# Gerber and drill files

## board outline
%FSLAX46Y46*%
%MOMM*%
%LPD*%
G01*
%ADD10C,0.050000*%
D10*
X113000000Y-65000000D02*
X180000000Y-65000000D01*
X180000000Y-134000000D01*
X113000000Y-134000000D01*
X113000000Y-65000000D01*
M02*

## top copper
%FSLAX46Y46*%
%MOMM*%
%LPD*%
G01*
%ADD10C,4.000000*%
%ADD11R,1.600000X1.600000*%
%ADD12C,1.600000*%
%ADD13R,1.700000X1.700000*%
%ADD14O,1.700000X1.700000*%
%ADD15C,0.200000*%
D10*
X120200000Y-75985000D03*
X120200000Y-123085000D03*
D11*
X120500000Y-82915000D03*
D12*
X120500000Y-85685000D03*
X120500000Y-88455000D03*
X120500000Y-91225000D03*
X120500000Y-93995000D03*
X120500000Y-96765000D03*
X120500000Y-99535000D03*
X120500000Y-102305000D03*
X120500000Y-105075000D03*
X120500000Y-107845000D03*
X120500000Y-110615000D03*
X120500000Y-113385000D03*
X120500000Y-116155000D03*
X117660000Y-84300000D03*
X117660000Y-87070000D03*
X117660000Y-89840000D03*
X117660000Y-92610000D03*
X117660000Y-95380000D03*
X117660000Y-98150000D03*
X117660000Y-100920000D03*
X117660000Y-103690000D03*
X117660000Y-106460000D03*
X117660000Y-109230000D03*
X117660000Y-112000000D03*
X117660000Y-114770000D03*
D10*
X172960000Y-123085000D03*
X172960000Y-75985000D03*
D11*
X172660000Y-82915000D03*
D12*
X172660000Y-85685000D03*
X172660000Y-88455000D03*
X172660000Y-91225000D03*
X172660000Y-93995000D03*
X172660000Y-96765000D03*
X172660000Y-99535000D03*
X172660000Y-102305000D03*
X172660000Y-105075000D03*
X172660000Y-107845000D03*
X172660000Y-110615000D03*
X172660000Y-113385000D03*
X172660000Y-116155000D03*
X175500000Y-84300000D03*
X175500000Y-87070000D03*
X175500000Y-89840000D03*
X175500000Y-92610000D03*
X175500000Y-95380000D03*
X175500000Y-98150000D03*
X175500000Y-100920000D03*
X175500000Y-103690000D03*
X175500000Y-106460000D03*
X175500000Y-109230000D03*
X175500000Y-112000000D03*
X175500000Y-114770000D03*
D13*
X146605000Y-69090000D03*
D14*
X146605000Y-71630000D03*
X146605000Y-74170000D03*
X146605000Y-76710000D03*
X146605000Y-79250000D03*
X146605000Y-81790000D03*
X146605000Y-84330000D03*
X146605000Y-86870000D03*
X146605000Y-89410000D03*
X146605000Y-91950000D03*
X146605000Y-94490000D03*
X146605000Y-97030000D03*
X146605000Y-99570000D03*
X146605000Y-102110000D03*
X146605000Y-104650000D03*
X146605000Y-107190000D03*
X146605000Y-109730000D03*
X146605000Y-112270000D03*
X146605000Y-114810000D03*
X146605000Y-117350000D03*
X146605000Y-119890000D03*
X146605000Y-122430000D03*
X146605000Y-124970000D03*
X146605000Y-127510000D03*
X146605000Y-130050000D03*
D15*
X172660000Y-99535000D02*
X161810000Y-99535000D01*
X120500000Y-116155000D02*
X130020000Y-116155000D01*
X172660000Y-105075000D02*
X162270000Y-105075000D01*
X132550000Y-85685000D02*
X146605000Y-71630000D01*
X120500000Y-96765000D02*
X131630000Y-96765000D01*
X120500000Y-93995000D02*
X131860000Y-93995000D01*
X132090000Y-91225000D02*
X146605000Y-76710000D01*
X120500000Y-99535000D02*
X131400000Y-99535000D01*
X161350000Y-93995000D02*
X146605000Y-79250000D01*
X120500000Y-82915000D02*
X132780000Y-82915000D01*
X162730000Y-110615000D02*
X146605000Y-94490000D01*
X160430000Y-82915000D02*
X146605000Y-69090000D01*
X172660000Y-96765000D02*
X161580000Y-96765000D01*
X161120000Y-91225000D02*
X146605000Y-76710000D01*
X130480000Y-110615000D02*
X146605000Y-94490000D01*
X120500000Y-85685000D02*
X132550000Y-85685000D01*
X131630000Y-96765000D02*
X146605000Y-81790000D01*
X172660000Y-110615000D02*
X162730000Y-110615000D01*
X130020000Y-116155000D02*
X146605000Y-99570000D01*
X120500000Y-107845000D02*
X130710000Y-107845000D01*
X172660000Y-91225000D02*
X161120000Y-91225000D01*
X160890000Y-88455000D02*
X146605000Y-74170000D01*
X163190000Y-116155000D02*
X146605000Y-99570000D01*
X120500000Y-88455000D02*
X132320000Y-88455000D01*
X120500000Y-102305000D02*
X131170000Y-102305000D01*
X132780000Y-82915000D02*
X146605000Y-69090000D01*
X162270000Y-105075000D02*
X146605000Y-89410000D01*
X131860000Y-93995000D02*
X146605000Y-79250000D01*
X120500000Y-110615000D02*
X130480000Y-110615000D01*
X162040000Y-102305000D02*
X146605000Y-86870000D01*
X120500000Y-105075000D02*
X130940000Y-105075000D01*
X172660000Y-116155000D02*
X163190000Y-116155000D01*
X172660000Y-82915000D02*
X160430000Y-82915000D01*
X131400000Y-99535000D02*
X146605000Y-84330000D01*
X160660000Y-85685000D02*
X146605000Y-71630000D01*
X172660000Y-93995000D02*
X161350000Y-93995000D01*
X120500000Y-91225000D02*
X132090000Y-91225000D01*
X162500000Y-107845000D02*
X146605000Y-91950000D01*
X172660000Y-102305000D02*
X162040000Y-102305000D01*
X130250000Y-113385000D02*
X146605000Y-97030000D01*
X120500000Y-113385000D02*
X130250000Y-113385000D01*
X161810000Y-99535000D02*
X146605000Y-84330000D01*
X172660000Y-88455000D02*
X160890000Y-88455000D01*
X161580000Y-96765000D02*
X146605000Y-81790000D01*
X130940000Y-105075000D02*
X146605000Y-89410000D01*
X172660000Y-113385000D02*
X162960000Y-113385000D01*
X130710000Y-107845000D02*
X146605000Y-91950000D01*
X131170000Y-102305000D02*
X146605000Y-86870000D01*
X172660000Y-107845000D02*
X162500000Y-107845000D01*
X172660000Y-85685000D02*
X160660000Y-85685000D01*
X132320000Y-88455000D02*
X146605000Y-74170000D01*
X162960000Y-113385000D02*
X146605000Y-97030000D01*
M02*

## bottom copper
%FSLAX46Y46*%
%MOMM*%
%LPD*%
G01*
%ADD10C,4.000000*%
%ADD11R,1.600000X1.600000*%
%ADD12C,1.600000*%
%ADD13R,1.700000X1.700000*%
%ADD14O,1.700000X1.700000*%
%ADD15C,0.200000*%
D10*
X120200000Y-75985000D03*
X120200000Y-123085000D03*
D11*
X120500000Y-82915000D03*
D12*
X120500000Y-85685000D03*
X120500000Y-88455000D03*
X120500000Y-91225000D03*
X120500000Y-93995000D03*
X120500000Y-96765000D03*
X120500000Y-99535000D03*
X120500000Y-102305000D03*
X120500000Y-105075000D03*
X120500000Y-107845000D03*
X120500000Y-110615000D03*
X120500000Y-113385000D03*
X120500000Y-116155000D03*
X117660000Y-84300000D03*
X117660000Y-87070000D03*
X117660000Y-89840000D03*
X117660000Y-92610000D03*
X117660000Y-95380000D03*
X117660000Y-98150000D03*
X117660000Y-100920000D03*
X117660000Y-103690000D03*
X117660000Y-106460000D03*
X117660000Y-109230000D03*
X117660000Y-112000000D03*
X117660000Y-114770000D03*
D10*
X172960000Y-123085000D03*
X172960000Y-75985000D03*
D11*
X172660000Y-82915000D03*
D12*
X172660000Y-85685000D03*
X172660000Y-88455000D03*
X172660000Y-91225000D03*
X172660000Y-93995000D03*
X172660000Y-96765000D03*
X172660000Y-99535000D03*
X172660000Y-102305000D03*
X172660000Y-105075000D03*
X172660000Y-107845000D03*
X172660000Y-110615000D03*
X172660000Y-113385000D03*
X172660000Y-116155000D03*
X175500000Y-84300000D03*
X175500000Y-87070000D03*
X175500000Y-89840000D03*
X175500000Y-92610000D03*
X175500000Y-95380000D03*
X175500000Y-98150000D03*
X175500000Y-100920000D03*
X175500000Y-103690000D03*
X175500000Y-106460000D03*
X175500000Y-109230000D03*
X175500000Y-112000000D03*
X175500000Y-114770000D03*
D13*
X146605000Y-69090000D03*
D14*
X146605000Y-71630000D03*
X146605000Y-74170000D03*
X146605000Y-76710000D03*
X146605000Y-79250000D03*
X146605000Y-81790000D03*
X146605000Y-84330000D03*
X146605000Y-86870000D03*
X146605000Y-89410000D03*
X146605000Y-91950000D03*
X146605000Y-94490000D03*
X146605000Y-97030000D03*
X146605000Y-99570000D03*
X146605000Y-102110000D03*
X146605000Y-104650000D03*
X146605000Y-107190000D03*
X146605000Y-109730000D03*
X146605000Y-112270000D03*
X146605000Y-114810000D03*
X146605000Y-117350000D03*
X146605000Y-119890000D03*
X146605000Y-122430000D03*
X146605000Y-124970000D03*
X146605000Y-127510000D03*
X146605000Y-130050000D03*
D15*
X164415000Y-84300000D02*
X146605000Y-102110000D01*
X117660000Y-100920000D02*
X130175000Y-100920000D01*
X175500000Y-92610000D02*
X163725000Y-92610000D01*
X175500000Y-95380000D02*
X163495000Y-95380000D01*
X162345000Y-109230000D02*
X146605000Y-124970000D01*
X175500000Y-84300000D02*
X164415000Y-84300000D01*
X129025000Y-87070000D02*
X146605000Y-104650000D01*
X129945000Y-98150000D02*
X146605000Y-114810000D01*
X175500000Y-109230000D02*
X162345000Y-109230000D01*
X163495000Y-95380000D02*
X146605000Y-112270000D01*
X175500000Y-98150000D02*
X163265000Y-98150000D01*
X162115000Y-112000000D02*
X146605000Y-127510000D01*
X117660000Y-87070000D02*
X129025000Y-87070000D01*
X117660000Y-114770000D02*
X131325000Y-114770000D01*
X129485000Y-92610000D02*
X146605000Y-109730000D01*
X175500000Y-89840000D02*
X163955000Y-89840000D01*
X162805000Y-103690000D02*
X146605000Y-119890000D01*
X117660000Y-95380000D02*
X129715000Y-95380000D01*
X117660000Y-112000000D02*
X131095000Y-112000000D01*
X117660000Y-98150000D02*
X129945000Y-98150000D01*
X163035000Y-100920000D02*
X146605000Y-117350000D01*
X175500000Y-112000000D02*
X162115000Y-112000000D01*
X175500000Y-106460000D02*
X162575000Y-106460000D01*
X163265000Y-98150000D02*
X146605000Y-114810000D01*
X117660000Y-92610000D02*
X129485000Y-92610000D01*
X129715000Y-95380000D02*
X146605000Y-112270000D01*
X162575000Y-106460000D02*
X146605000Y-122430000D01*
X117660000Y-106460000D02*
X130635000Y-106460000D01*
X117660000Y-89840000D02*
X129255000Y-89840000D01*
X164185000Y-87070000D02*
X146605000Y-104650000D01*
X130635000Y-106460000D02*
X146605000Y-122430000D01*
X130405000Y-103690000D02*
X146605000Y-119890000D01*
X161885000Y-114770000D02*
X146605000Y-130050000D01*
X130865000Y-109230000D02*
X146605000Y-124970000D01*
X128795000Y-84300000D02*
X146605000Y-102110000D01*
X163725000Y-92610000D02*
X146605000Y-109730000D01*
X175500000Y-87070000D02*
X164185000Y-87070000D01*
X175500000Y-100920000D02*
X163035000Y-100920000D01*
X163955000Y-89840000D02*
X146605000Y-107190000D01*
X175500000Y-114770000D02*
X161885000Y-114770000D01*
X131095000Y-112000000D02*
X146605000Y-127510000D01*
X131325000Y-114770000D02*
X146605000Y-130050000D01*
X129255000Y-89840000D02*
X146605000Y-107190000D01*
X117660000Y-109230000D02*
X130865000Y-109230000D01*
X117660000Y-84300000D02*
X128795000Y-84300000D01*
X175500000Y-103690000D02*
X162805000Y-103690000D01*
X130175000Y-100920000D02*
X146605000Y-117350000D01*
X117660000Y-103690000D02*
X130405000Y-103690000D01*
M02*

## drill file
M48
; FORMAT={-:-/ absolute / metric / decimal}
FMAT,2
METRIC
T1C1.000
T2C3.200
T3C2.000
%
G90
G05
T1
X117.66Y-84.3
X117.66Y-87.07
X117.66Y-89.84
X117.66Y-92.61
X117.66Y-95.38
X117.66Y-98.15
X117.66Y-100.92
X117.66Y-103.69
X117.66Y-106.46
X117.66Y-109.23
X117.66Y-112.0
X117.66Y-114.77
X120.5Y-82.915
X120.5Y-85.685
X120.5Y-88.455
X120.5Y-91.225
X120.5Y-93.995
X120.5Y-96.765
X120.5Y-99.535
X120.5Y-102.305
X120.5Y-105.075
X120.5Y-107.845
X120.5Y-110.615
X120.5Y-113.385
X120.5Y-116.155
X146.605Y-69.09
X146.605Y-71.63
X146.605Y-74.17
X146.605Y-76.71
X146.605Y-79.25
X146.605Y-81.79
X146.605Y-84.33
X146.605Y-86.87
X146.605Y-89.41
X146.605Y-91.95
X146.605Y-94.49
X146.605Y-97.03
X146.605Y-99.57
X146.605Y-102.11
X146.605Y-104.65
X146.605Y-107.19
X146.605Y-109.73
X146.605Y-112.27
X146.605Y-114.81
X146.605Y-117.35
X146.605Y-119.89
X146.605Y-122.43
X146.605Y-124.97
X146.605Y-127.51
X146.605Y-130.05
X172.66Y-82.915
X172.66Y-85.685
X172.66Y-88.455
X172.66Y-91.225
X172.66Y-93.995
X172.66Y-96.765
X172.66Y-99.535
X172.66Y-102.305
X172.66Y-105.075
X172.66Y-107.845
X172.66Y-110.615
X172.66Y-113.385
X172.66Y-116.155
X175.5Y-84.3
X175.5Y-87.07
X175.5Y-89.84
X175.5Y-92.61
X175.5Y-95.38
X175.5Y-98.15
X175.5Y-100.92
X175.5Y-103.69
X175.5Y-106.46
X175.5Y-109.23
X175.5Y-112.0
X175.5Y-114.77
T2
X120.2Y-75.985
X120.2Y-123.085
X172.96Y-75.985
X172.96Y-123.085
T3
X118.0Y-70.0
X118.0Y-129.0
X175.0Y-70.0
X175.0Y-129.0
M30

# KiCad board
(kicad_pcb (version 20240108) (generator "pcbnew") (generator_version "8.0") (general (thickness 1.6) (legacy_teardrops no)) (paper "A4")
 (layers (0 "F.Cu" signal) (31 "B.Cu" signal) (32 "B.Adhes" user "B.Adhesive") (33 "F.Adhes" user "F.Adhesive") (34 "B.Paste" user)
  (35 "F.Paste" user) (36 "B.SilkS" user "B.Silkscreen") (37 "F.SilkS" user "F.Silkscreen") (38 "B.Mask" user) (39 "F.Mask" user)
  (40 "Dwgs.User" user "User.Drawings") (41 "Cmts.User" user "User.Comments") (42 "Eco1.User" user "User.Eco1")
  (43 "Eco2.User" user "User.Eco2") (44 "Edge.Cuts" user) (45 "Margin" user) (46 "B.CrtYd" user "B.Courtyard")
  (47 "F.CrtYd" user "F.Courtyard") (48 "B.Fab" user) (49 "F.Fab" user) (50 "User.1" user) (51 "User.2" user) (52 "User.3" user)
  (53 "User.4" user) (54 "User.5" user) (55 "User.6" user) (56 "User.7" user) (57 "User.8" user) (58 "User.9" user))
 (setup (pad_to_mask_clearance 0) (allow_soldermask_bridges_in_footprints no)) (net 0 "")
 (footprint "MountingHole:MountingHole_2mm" (layer "F.Cu") (at 175 70)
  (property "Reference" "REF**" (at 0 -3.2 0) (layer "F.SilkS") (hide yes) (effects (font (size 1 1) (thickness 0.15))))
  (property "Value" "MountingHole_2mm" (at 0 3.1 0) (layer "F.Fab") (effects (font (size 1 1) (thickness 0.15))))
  (pad "" np_thru_hole circle (at 0 0) (size 2 2) (drill 2) (layers "*.Cu" "*.Mask")))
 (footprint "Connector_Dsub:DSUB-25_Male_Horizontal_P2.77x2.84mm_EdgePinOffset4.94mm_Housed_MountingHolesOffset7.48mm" (layer "F.Cu")
  (at 120.5 82.915 -90)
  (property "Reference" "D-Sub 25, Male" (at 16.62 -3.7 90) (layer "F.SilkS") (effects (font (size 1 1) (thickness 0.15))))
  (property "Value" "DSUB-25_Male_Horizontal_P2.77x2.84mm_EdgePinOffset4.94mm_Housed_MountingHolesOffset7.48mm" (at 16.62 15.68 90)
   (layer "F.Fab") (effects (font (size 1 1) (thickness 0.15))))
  (pad "0" thru_hole circle (at -6.93 0.3 270) (size 4 4) (drill 3.2) (layers "*.Cu" "*.Mask") (remove_unused_layers no))
  (pad "0" thru_hole circle (at 40.17 0.3 270) (size 4 4) (drill 3.2) (layers "*.Cu" "*.Mask") (remove_unused_layers no))
  (pad "1" thru_hole rect (at 0 0 270) (size 1.6 1.6) (drill 1) (layers "*.Cu" "*.Mask") (remove_unused_layers no))
  (pad "2" thru_hole circle (at 2.77 0 270) (size 1.6 1.6) (drill 1) (layers "*.Cu" "*.Mask") (remove_unused_layers no))
  (pad "3" thru_hole circle (at 5.54 0 270) (size 1.6 1.6) (drill 1) (layers "*.Cu" "*.Mask") (remove_unused_layers no))
  (pad "4" thru_hole circle (at 8.31 0 270) (size 1.6 1.6) (drill 1) (layers "*.Cu" "*.Mask") (remove_unused_layers no))
  (pad "5" thru_hole circle (at 11.08 0 270) (size 1.6 1.6) (drill 1) (layers "*.Cu" "*.Mask") (remove_unused_layers no))
  (pad "6" thru_hole circle (at 13.85 0 270) (size 1.6 1.6) (drill 1) (layers "*.Cu" "*.Mask") (remove_unused_layers no))
  (pad "7" thru_hole circle (at 16.62 0 270) (size 1.6 1.6) (drill 1) (layers "*.Cu" "*.Mask") (remove_unused_layers no))
  (pad "8" thru_hole circle (at 19.39 0 270) (size 1.6 1.6) (drill 1) (layers "*.Cu" "*.Mask") (remove_unused_layers no))
  (pad "9" thru_hole circle (at 22.16 0 270) (size 1.6 1.6) (drill 1) (layers "*.Cu" "*.Mask") (remove_unused_layers no))
  (pad "10" thru_hole circle (at 24.93 0 270) (size 1.6 1.6) (drill 1) (layers "*.Cu" "*.Mask") (remove_unused_layers no))
  (pad "11" thru_hole circle (at 27.7 0 270) (size 1.6 1.6) (drill 1) (layers "*.Cu" "*.Mask") (remove_unused_layers no))
  (pad "12" thru_hole circle (at 30.47 0 270) (size 1.6 1.6) (drill 1) (layers "*.Cu" "*.Mask") (remove_unused_layers no))
  (pad "13" thru_hole circle (at 33.24 0 270) (size 1.6 1.6) (drill 1) (layers "*.Cu" "*.Mask") (remove_unused_layers no))
  (pad "14" thru_hole circle (at 1.385 2.84 270) (size 1.6 1.6) (drill 1) (layers "*.Cu" "*.Mask") (remove_unused_layers no))
  (pad "15" thru_hole circle (at 4.155 2.84 270) (size 1.6 1.6) (drill 1) (layers "*.Cu" "*.Mask") (remove_unused_layers no))
  (pad "16" thru_hole circle (at 6.925 2.84 270) (size 1.6 1.6) (drill 1) (layers "*.Cu" "*.Mask") (remove_unused_layers no))
  (pad "17" thru_hole circle (at 9.695 2.84 270) (size 1.6 1.6) (drill 1) (layers "*.Cu" "*.Mask") (remove_unused_layers no))
  (pad "18" thru_hole circle (at 12.465 2.84 270) (size 1.6 1.6) (drill 1) (layers "*.Cu" "*.Mask") (remove_unused_layers no))
  (pad "19" thru_hole circle (at 15.235 2.84 270) (size 1.6 1.6) (drill 1) (layers "*.Cu" "*.Mask") (remove_unused_layers no))
  (pad "20" thru_hole circle (at 18.005 2.84 270) (size 1.6 1.6) (drill 1) (layers "*.Cu" "*.Mask") (remove_unused_layers no))
  (pad "21" thru_hole circle (at 20.775 2.84 270) (size 1.6 1.6) (drill 1) (layers "*.Cu" "*.Mask") (remove_unused_layers no))
  (pad "22" thru_hole circle (at 23.545 2.84 270) (size 1.6 1.6) (drill 1) (layers "*.Cu" "*.Mask") (remove_unused_layers no))
  (pad "23" thru_hole circle (at 26.315 2.84 270) (size 1.6 1.6) (drill 1) (layers "*.Cu" "*.Mask") (remove_unused_layers no))
  (pad "24" thru_hole circle (at 29.085 2.84 270) (size 1.6 1.6) (drill 1) (layers "*.Cu" "*.Mask") (remove_unused_layers no))
  (pad "25" thru_hole circle (at 31.855 2.84 270) (size 1.6 1.6) (drill 1) (layers "*.Cu" "*.Mask") (remove_unused_layers no)))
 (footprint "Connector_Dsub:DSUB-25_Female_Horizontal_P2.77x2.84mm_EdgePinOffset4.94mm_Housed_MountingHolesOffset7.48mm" (layer "F.Cu")
  (at 172.66 82.915 90)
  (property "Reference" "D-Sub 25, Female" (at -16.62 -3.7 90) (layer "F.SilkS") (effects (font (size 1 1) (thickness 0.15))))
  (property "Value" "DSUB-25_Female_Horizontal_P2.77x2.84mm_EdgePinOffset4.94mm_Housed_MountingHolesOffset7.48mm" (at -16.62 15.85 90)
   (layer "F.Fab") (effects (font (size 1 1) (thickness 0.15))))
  (pad "0" thru_hole circle (at -40.17 0.3 90) (size 4 4) (drill 3.2) (layers "*.Cu" "*.Mask") (remove_unused_layers no))
  (pad "0" thru_hole circle (at 6.93 0.3 90) (size 4 4) (drill 3.2) (layers "*.Cu" "*.Mask") (remove_unused_layers no))
  (pad "1" thru_hole rect (at 0 0 90) (size 1.6 1.6) (drill 1) (layers "*.Cu" "*.Mask") (remove_unused_layers no))
  (pad "2" thru_hole circle (at -2.77 0 90) (size 1.6 1.6) (drill 1) (layers "*.Cu" "*.Mask") (remove_unused_layers no))
  (pad "3" thru_hole circle (at -5.54 0 90) (size 1.6 1.6) (drill 1) (layers "*.Cu" "*.Mask") (remove_unused_layers no))
  (pad "4" thru_hole circle (at -8.31 0 90) (size 1.6 1.6) (drill 1) (layers "*.Cu" "*.Mask") (remove_unused_layers no))
  (pad "5" thru_hole circle (at -11.08 0 90) (size 1.6 1.6) (drill 1) (layers "*.Cu" "*.Mask") (remove_unused_layers no))
  (pad "6" thru_hole circle (at -13.85 0 90) (size 1.6 1.6) (drill 1) (layers "*.Cu" "*.Mask") (remove_unused_layers no))
  (pad "7" thru_hole circle (at -16.62 0 90) (size 1.6 1.6) (drill 1) (layers "*.Cu" "*.Mask") (remove_unused_layers no))
  (pad "8" thru_hole circle (at -19.39 0 90) (size 1.6 1.6) (drill 1) (layers "*.Cu" "*.Mask") (remove_unused_layers no))
  (pad "9" thru_hole circle (at -22.16 0 90) (size 1.6 1.6) (drill 1) (layers "*.Cu" "*.Mask") (remove_unused_layers no))
  (pad "10" thru_hole circle (at -24.93 0 90) (size 1.6 1.6) (drill 1) (layers "*.Cu" "*.Mask") (remove_unused_layers no))
  (pad "11" thru_hole circle (at -27.7 0 90) (size 1.6 1.6) (drill 1) (layers "*.Cu" "*.Mask") (remove_unused_layers no))
  (pad "12" thru_hole circle (at -30.47 0 90) (size 1.6 1.6) (drill 1) (layers "*.Cu" "*.Mask") (remove_unused_layers no))
  (pad "13" thru_hole circle (at -33.24 0 90) (size 1.6 1.6) (drill 1) (layers "*.Cu" "*.Mask") (remove_unused_layers no))
  (pad "14" thru_hole circle (at -1.385 2.84 90) (size 1.6 1.6) (drill 1) (layers "*.Cu" "*.Mask") (remove_unused_layers no))
  (pad "15" thru_hole circle (at -4.155 2.84 90) (size 1.6 1.6) (drill 1) (layers "*.Cu" "*.Mask") (remove_unused_layers no))
  (pad "16" thru_hole circle (at -6.925 2.84 90) (size 1.6 1.6) (drill 1) (layers "*.Cu" "*.Mask") (remove_unused_layers no))
  (pad "17" thru_hole circle (at -9.695 2.84 90) (size 1.6 1.6) (drill 1) (layers "*.Cu" "*.Mask") (remove_unused_layers no))
  (pad "18" thru_hole circle (at -12.465 2.84 90) (size 1.6 1.6) (drill 1) (layers "*.Cu" "*.Mask") (remove_unused_layers no))
  (pad "19" thru_hole circle (at -15.235 2.84 90) (size 1.6 1.6) (drill 1) (layers "*.Cu" "*.Mask") (remove_unused_layers no))
  (pad "20" thru_hole circle (at -18.005 2.84 90) (size 1.6 1.6) (drill 1) (layers "*.Cu" "*.Mask") (remove_unused_layers no))
  (pad "21" thru_hole circle (at -20.775 2.84 90) (size 1.6 1.6) (drill 1) (layers "*.Cu" "*.Mask") (remove_unused_layers no))
  (pad "22" thru_hole circle (at -23.545 2.84 90) (size 1.6 1.6) (drill 1) (layers "*.Cu" "*.Mask") (remove_unused_layers no))
  (pad "23" thru_hole circle (at -26.315 2.84 90) (size 1.6 1.6) (drill 1) (layers "*.Cu" "*.Mask") (remove_unused_layers no))
  (pad "24" thru_hole circle (at -29.085 2.84 90) (size 1.6 1.6) (drill 1) (layers "*.Cu" "*.Mask") (remove_unused_layers no))
  (pad "25" thru_hole circle (at -31.855 2.84 90) (size 1.6 1.6) (drill 1) (layers "*.Cu" "*.Mask") (remove_unused_layers no)))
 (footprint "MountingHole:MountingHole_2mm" (layer "F.Cu") (at 175 129)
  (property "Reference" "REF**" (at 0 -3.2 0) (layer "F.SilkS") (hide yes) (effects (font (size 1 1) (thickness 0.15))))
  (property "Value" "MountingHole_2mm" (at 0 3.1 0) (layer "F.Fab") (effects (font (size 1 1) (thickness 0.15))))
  (pad "" np_thru_hole circle (at 0 0) (size 2 2) (drill 2) (layers "*.Cu" "*.Mask")))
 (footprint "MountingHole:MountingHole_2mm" (layer "F.Cu") (at 118 70)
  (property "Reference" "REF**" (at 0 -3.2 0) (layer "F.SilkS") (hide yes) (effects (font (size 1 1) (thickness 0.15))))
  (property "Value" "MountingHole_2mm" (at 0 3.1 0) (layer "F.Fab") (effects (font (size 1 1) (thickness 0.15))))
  (pad "" np_thru_hole circle (at 0 0) (size 2 2) (drill 2) (layers "*.Cu" "*.Mask")))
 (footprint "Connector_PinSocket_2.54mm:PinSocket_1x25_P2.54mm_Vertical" (layer "F.Cu") (at 146.605 69.09)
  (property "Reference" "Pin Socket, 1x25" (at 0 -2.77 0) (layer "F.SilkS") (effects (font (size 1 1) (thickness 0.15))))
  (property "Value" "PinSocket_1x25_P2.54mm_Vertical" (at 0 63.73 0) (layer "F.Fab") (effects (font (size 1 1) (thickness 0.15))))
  (pad "1" thru_hole rect (at 0 0) (size 1.7 1.7) (drill 1) (layers "*.Cu" "*.Mask") (remove_unused_layers no))
  (pad "2" thru_hole oval (at 0 2.54) (size 1.7 1.7) (drill 1) (layers "*.Cu" "*.Mask") (remove_unused_layers no))
  (pad "3" thru_hole oval (at 0 5.08) (size 1.7 1.7) (drill 1) (layers "*.Cu" "*.Mask") (remove_unused_layers no))
  (pad "4" thru_hole oval (at 0 7.62) (size 1.7 1.7) (drill 1) (layers "*.Cu" "*.Mask") (remove_unused_layers no))
  (pad "5" thru_hole oval (at 0 10.16) (size 1.7 1.7) (drill 1) (layers "*.Cu" "*.Mask") (remove_unused_layers no))
  (pad "6" thru_hole oval (at 0 12.7) (size 1.7 1.7) (drill 1) (layers "*.Cu" "*.Mask") (remove_unused_layers no))
  (pad "7" thru_hole oval (at 0 15.24) (size 1.7 1.7) (drill 1) (layers "*.Cu" "*.Mask") (remove_unused_layers no))
  (pad "8" thru_hole oval (at 0 17.78) (size 1.7 1.7) (drill 1) (layers "*.Cu" "*.Mask") (remove_unused_layers no))
  (pad "9" thru_hole oval (at 0 20.32) (size 1.7 1.7) (drill 1) (layers "*.Cu" "*.Mask") (remove_unused_layers no))
  (pad "10" thru_hole oval (at 0 22.86) (size 1.7 1.7) (drill 1) (layers "*.Cu" "*.Mask") (remove_unused_layers no))
  (pad "11" thru_hole oval (at 0 25.4) (size 1.7 1.7) (drill 1) (layers "*.Cu" "*.Mask") (remove_unused_layers no))
  (pad "12" thru_hole oval (at 0 27.94) (size 1.7 1.7) (drill 1) (layers "*.Cu" "*.Mask") (remove_unused_layers no))
  (pad "13" thru_hole oval (at 0 30.48) (size 1.7 1.7) (drill 1) (layers "*.Cu" "*.Mask") (remove_unused_layers no))
  (pad "14" thru_hole oval (at 0 33.02) (size 1.7 1.7) (drill 1) (layers "*.Cu" "*.Mask") (remove_unused_layers no))
  (pad "15" thru_hole oval (at 0 35.56) (size 1.7 1.7) (drill 1) (layers "*.Cu" "*.Mask") (remove_unused_layers no))
  (pad "16" thru_hole oval (at 0 38.1) (size 1.7 1.7) (drill 1) (layers "*.Cu" "*.Mask") (remove_unused_layers no))
  (pad "17" thru_hole oval (at 0 40.64) (size 1.7 1.7) (drill 1) (layers "*.Cu" "*.Mask") (remove_unused_layers no))
  (pad "18" thru_hole oval (at 0 43.18) (size 1.7 1.7) (drill 1) (layers "*.Cu" "*.Mask") (remove_unused_layers no))
  (pad "19" thru_hole oval (at 0 45.72) (size 1.7 1.7) (drill 1) (layers "*.Cu" "*.Mask") (remove_unused_layers no))
  (pad "20" thru_hole oval (at 0 48.26) (size 1.7 1.7) (drill 1) (layers "*.Cu" "*.Mask") (remove_unused_layers no))
  (pad "21" thru_hole oval (at 0 50.8) (size 1.7 1.7) (drill 1) (layers "*.Cu" "*.Mask") (remove_unused_layers no))
  (pad "22" thru_hole oval (at 0 53.34) (size 1.7 1.7) (drill 1) (layers "*.Cu" "*.Mask") (remove_unused_layers no))
  (pad "23" thru_hole oval (at 0 55.88) (size 1.7 1.7) (drill 1) (layers "*.Cu" "*.Mask") (remove_unused_layers no))
  (pad "24" thru_hole oval (at 0 58.42) (size 1.7 1.7) (drill 1) (layers "*.Cu" "*.Mask") (remove_unused_layers no))
  (pad "25" thru_hole oval (at 0 60.96) (size 1.7 1.7) (drill 1) (layers "*.Cu" "*.Mask") (remove_unused_layers no)))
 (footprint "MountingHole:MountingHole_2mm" (layer "F.Cu") (at 118 129)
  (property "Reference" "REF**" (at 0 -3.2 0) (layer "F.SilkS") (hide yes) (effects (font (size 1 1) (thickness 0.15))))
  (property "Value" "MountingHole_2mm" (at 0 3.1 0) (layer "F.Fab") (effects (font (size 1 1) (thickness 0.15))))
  (pad "" np_thru_hole circle (at 0 0) (size 2 2) (drill 2) (layers "*.Cu" "*.Mask")))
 (gr_rect (start 113 65) (end 180 134) (stroke (width 0.05) (type default)) (fill none) (layer "Edge.Cuts"))
 (segment (start 172.66 99.535) (end 161.81 99.535) (width 0.2) (layer "F.Cu") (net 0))
 (segment (start 120.5 116.155) (end 130.02 116.155) (width 0.2) (layer "F.Cu") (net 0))
 (segment (start 172.66 105.075) (end 162.27 105.075) (width 0.2) (layer "F.Cu") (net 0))
 (segment (start 132.55 85.685) (end 146.605 71.63) (width 0.2) (layer "F.Cu") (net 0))
 (segment (start 120.5 96.765) (end 131.63 96.765) (width 0.2) (layer "F.Cu") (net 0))
 (segment (start 120.5 93.995) (end 131.86 93.995) (width 0.2) (layer "F.Cu") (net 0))
 (segment (start 132.09 91.225) (end 146.605 76.71) (width 0.2) (layer "F.Cu") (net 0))
 (segment (start 120.5 99.535) (end 131.4 99.535) (width 0.2) (layer "F.Cu") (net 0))
 (segment (start 161.35 93.995) (end 146.605 79.25) (width 0.2) (layer "F.Cu") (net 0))
 (segment (start 120.5 82.915) (end 132.78 82.915) (width 0.2) (layer "F.Cu") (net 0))
 (segment (start 162.73 110.615) (end 146.605 94.49) (width 0.2) (layer "F.Cu") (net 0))
 (segment (start 160.43 82.915) (end 146.605 69.09) (width 0.2) (layer "F.Cu") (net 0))
 (segment (start 172.66 96.765) (end 161.58 96.765) (width 0.2) (layer "F.Cu") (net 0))
 (segment (start 161.12 91.225) (end 146.605 76.71) (width 0.2) (layer "F.Cu") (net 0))
 (segment (start 130.48 110.615) (end 146.605 94.49) (width 0.2) (layer "F.Cu") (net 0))
 (segment (start 120.5 85.685) (end 132.55 85.685) (width 0.2) (layer "F.Cu") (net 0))
 (segment (start 131.63 96.765) (end 146.605 81.79) (width 0.2) (layer "F.Cu") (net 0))
 (segment (start 172.66 110.615) (end 162.73 110.615) (width 0.2) (layer "F.Cu") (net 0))
 (segment (start 130.02 116.155) (end 146.605 99.57) (width 0.2) (layer "F.Cu") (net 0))
 (segment (start 120.5 107.845) (end 130.71 107.845) (width 0.2) (layer "F.Cu") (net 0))
 (segment (start 172.66 91.225) (end 161.12 91.225) (width 0.2) (layer "F.Cu") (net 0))
 (segment (start 160.89 88.455) (end 146.605 74.17) (width 0.2) (layer "F.Cu") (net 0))
 (segment (start 163.19 116.155) (end 146.605 99.57) (width 0.2) (layer "F.Cu") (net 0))
 (segment (start 120.5 88.455) (end 132.32 88.455) (width 0.2) (layer "F.Cu") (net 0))
 (segment (start 120.5 102.305) (end 131.17 102.305) (width 0.2) (layer "F.Cu") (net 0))
 (segment (start 132.78 82.915) (end 146.605 69.09) (width 0.2) (layer "F.Cu") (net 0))
 (segment (start 162.27 105.075) (end 146.605 89.41) (width 0.2) (layer "F.Cu") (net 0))
 (segment (start 131.86 93.995) (end 146.605 79.25) (width 0.2) (layer "F.Cu") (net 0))
 (segment (start 120.5 110.615) (end 130.48 110.615) (width 0.2) (layer "F.Cu") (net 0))
 (segment (start 162.04 102.305) (end 146.605 86.87) (width 0.2) (layer "F.Cu") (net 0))
 (segment (start 120.5 105.075) (end 130.94 105.075) (width 0.2) (layer "F.Cu") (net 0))
 (segment (start 172.66 116.155) (end 163.19 116.155) (width 0.2) (layer "F.Cu") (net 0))
 (segment (start 172.66 82.915) (end 160.43 82.915) (width 0.2) (layer "F.Cu") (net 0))
 (segment (start 131.4 99.535) (end 146.605 84.33) (width 0.2) (layer "F.Cu") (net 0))
 (segment (start 160.66 85.685) (end 146.605 71.63) (width 0.2) (layer "F.Cu") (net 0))
 (segment (start 172.66 93.995) (end 161.35 93.995) (width 0.2) (layer "F.Cu") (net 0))
 (segment (start 120.5 91.225) (end 132.09 91.225) (width 0.2) (layer "F.Cu") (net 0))
 (segment (start 162.5 107.845) (end 146.605 91.95) (width 0.2) (layer "F.Cu") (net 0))
 (segment (start 172.66 102.305) (end 162.04 102.305) (width 0.2) (layer "F.Cu") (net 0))
 (segment (start 130.25 113.385) (end 146.605 97.03) (width 0.2) (layer "F.Cu") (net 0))
 (segment (start 120.5 113.385) (end 130.25 113.385) (width 0.2) (layer "F.Cu") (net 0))
 (segment (start 161.81 99.535) (end 146.605 84.33) (width 0.2) (layer "F.Cu") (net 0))
 (segment (start 172.66 88.455) (end 160.89 88.455) (width 0.2) (layer "F.Cu") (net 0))
 (segment (start 161.58 96.765) (end 146.605 81.79) (width 0.2) (layer "F.Cu") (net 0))
 (segment (start 130.94 105.075) (end 146.605 89.41) (width 0.2) (layer "F.Cu") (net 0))
 (segment (start 172.66 113.385) (end 162.96 113.385) (width 0.2) (layer "F.Cu") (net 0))
 (segment (start 130.71 107.845) (end 146.605 91.95) (width 0.2) (layer "F.Cu") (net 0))
 (segment (start 131.17 102.305) (end 146.605 86.87) (width 0.2) (layer "F.Cu") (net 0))
 (segment (start 172.66 107.845) (end 162.5 107.845) (width 0.2) (layer "F.Cu") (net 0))
 (segment (start 172.66 85.685) (end 160.66 85.685) (width 0.2) (layer "F.Cu") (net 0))
 (segment (start 132.32 88.455) (end 146.605 74.17) (width 0.2) (layer "F.Cu") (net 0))
 (segment (start 162.96 113.385) (end 146.605 97.03) (width 0.2) (layer "F.Cu") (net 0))
 (segment (start 164.415 84.3) (end 146.605 102.11) (width 0.2) (layer "B.Cu") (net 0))
 (segment (start 117.66 100.92) (end 130.175 100.92) (width 0.2) (layer "B.Cu") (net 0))
 (segment (start 175.5 92.61) (end 163.725 92.61) (width 0.2) (layer "B.Cu") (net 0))
 (segment (start 175.5 95.38) (end 163.495 95.38) (width 0.2) (layer "B.Cu") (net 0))
 (segment (start 162.345 109.23) (end 146.605 124.97) (width 0.2) (layer "B.Cu") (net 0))
 (segment (start 175.5 84.3) (end 164.415 84.3) (width 0.2) (layer "B.Cu") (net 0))
 (segment (start 129.025 87.07) (end 146.605 104.65) (width 0.2) (layer "B.Cu") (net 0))
 (segment (start 129.945 98.15) (end 146.605 114.81) (width 0.2) (layer "B.Cu") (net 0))
 (segment (start 175.5 109.23) (end 162.345 109.23) (width 0.2) (layer "B.Cu") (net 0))
 (segment (start 163.495 95.38) (end 146.605 112.27) (width 0.2) (layer "B.Cu") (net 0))
 (segment (start 175.5 98.15) (end 163.265 98.15) (width 0.2) (layer "B.Cu") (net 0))
 (segment (start 162.115 112) (end 146.605 127.51) (width 0.2) (layer "B.Cu") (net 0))
 (segment (start 117.66 87.07) (end 129.025 87.07) (width 0.2) (layer "B.Cu") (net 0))
 (segment (start 117.66 114.77) (end 131.325 114.77) (width 0.2) (layer "B.Cu") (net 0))
 (segment (start 129.485 92.61) (end 146.605 109.73) (width 0.2) (layer "B.Cu") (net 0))
 (segment (start 175.5 89.84) (end 163.955 89.84) (width 0.2) (layer "B.Cu") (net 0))
 (segment (start 162.805 103.69) (end 146.605 119.89) (width 0.2) (layer "B.Cu") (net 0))
 (segment (start 117.66 95.38) (end 129.715 95.38) (width 0.2) (layer "B.Cu") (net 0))
 (segment (start 117.66 112) (end 131.095 112) (width 0.2) (layer "B.Cu") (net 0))
 (segment (start 117.66 98.15) (end 129.945 98.15) (width 0.2) (layer "B.Cu") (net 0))
 (segment (start 163.035 100.92) (end 146.605 117.35) (width 0.2) (layer "B.Cu") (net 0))
 (segment (start 175.5 112) (end 162.115 112) (width 0.2) (layer "B.Cu") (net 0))
 (segment (start 175.5 106.46) (end 162.575 106.46) (width 0.2) (layer "B.Cu") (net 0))
 (segment (start 163.265 98.15) (end 146.605 114.81) (width 0.2) (layer "B.Cu") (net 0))
 (segment (start 117.66 92.61) (end 129.485 92.61) (width 0.2) (layer "B.Cu") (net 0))
 (segment (start 129.715 95.38) (end 146.605 112.27) (width 0.2) (layer "B.Cu") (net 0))
 (segment (start 162.575 106.46) (end 146.605 122.43) (width 0.2) (layer "B.Cu") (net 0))
 (segment (start 117.66 106.46) (end 130.635 106.46) (width 0.2) (layer "B.Cu") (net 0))
 (segment (start 117.66 89.84) (end 129.255 89.84) (width 0.2) (layer "B.Cu") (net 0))
 (segment (start 164.185 87.07) (end 146.605 104.65) (width 0.2) (layer "B.Cu") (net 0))
 (segment (start 130.635 106.46) (end 146.605 122.43) (width 0.2) (layer "B.Cu") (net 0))
 (segment (start 130.405 103.69) (end 146.605 119.89) (width 0.2) (layer "B.Cu") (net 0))
 (segment (start 161.885 114.77) (end 146.605 130.05) (width 0.2) (layer "B.Cu") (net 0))
 (segment (start 130.865 109.23) (end 146.605 124.97) (width 0.2) (layer "B.Cu") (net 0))
 (segment (start 128.795 84.3) (end 146.605 102.11) (width 0.2) (layer "B.Cu") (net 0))
 (segment (start 163.725 92.61) (end 146.605 109.73) (width 0.2) (layer "B.Cu") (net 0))
 (segment (start 175.5 87.07) (end 164.185 87.07) (width 0.2) (layer "B.Cu") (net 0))
 (segment (start 175.5 100.92) (end 163.035 100.92) (width 0.2) (layer "B.Cu") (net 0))
 (segment (start 163.955 89.84) (end 146.605 107.19) (width 0.2) (layer "B.Cu") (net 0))
 (segment (start 175.5 114.77) (end 161.885 114.77) (width 0.2) (layer "B.Cu") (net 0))
 (segment (start 131.095 112) (end 146.605 127.51) (width 0.2) (layer "B.Cu") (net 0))
 (segment (start 131.325 114.77) (end 146.605 130.05) (width 0.2) (layer "B.Cu") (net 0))
 (segment (start 129.255 89.84) (end 146.605 107.19) (width 0.2) (layer "B.Cu") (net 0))
 (segment (start 117.66 109.23) (end 130.865 109.23) (width 0.2) (layer "B.Cu") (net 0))
 (segment (start 117.66 84.3) (end 128.795 84.3) (width 0.2) (layer "B.Cu") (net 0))
 (segment (start 175.5 103.69) (end 162.805 103.69) (width 0.2) (layer "B.Cu") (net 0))
 (segment (start 130.175 100.92) (end 146.605 117.35) (width 0.2) (layer "B.Cu") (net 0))
 (segment (start 117.66 103.69) (end 130.405 103.69) (width 0.2) (layer "B.Cu") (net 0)))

